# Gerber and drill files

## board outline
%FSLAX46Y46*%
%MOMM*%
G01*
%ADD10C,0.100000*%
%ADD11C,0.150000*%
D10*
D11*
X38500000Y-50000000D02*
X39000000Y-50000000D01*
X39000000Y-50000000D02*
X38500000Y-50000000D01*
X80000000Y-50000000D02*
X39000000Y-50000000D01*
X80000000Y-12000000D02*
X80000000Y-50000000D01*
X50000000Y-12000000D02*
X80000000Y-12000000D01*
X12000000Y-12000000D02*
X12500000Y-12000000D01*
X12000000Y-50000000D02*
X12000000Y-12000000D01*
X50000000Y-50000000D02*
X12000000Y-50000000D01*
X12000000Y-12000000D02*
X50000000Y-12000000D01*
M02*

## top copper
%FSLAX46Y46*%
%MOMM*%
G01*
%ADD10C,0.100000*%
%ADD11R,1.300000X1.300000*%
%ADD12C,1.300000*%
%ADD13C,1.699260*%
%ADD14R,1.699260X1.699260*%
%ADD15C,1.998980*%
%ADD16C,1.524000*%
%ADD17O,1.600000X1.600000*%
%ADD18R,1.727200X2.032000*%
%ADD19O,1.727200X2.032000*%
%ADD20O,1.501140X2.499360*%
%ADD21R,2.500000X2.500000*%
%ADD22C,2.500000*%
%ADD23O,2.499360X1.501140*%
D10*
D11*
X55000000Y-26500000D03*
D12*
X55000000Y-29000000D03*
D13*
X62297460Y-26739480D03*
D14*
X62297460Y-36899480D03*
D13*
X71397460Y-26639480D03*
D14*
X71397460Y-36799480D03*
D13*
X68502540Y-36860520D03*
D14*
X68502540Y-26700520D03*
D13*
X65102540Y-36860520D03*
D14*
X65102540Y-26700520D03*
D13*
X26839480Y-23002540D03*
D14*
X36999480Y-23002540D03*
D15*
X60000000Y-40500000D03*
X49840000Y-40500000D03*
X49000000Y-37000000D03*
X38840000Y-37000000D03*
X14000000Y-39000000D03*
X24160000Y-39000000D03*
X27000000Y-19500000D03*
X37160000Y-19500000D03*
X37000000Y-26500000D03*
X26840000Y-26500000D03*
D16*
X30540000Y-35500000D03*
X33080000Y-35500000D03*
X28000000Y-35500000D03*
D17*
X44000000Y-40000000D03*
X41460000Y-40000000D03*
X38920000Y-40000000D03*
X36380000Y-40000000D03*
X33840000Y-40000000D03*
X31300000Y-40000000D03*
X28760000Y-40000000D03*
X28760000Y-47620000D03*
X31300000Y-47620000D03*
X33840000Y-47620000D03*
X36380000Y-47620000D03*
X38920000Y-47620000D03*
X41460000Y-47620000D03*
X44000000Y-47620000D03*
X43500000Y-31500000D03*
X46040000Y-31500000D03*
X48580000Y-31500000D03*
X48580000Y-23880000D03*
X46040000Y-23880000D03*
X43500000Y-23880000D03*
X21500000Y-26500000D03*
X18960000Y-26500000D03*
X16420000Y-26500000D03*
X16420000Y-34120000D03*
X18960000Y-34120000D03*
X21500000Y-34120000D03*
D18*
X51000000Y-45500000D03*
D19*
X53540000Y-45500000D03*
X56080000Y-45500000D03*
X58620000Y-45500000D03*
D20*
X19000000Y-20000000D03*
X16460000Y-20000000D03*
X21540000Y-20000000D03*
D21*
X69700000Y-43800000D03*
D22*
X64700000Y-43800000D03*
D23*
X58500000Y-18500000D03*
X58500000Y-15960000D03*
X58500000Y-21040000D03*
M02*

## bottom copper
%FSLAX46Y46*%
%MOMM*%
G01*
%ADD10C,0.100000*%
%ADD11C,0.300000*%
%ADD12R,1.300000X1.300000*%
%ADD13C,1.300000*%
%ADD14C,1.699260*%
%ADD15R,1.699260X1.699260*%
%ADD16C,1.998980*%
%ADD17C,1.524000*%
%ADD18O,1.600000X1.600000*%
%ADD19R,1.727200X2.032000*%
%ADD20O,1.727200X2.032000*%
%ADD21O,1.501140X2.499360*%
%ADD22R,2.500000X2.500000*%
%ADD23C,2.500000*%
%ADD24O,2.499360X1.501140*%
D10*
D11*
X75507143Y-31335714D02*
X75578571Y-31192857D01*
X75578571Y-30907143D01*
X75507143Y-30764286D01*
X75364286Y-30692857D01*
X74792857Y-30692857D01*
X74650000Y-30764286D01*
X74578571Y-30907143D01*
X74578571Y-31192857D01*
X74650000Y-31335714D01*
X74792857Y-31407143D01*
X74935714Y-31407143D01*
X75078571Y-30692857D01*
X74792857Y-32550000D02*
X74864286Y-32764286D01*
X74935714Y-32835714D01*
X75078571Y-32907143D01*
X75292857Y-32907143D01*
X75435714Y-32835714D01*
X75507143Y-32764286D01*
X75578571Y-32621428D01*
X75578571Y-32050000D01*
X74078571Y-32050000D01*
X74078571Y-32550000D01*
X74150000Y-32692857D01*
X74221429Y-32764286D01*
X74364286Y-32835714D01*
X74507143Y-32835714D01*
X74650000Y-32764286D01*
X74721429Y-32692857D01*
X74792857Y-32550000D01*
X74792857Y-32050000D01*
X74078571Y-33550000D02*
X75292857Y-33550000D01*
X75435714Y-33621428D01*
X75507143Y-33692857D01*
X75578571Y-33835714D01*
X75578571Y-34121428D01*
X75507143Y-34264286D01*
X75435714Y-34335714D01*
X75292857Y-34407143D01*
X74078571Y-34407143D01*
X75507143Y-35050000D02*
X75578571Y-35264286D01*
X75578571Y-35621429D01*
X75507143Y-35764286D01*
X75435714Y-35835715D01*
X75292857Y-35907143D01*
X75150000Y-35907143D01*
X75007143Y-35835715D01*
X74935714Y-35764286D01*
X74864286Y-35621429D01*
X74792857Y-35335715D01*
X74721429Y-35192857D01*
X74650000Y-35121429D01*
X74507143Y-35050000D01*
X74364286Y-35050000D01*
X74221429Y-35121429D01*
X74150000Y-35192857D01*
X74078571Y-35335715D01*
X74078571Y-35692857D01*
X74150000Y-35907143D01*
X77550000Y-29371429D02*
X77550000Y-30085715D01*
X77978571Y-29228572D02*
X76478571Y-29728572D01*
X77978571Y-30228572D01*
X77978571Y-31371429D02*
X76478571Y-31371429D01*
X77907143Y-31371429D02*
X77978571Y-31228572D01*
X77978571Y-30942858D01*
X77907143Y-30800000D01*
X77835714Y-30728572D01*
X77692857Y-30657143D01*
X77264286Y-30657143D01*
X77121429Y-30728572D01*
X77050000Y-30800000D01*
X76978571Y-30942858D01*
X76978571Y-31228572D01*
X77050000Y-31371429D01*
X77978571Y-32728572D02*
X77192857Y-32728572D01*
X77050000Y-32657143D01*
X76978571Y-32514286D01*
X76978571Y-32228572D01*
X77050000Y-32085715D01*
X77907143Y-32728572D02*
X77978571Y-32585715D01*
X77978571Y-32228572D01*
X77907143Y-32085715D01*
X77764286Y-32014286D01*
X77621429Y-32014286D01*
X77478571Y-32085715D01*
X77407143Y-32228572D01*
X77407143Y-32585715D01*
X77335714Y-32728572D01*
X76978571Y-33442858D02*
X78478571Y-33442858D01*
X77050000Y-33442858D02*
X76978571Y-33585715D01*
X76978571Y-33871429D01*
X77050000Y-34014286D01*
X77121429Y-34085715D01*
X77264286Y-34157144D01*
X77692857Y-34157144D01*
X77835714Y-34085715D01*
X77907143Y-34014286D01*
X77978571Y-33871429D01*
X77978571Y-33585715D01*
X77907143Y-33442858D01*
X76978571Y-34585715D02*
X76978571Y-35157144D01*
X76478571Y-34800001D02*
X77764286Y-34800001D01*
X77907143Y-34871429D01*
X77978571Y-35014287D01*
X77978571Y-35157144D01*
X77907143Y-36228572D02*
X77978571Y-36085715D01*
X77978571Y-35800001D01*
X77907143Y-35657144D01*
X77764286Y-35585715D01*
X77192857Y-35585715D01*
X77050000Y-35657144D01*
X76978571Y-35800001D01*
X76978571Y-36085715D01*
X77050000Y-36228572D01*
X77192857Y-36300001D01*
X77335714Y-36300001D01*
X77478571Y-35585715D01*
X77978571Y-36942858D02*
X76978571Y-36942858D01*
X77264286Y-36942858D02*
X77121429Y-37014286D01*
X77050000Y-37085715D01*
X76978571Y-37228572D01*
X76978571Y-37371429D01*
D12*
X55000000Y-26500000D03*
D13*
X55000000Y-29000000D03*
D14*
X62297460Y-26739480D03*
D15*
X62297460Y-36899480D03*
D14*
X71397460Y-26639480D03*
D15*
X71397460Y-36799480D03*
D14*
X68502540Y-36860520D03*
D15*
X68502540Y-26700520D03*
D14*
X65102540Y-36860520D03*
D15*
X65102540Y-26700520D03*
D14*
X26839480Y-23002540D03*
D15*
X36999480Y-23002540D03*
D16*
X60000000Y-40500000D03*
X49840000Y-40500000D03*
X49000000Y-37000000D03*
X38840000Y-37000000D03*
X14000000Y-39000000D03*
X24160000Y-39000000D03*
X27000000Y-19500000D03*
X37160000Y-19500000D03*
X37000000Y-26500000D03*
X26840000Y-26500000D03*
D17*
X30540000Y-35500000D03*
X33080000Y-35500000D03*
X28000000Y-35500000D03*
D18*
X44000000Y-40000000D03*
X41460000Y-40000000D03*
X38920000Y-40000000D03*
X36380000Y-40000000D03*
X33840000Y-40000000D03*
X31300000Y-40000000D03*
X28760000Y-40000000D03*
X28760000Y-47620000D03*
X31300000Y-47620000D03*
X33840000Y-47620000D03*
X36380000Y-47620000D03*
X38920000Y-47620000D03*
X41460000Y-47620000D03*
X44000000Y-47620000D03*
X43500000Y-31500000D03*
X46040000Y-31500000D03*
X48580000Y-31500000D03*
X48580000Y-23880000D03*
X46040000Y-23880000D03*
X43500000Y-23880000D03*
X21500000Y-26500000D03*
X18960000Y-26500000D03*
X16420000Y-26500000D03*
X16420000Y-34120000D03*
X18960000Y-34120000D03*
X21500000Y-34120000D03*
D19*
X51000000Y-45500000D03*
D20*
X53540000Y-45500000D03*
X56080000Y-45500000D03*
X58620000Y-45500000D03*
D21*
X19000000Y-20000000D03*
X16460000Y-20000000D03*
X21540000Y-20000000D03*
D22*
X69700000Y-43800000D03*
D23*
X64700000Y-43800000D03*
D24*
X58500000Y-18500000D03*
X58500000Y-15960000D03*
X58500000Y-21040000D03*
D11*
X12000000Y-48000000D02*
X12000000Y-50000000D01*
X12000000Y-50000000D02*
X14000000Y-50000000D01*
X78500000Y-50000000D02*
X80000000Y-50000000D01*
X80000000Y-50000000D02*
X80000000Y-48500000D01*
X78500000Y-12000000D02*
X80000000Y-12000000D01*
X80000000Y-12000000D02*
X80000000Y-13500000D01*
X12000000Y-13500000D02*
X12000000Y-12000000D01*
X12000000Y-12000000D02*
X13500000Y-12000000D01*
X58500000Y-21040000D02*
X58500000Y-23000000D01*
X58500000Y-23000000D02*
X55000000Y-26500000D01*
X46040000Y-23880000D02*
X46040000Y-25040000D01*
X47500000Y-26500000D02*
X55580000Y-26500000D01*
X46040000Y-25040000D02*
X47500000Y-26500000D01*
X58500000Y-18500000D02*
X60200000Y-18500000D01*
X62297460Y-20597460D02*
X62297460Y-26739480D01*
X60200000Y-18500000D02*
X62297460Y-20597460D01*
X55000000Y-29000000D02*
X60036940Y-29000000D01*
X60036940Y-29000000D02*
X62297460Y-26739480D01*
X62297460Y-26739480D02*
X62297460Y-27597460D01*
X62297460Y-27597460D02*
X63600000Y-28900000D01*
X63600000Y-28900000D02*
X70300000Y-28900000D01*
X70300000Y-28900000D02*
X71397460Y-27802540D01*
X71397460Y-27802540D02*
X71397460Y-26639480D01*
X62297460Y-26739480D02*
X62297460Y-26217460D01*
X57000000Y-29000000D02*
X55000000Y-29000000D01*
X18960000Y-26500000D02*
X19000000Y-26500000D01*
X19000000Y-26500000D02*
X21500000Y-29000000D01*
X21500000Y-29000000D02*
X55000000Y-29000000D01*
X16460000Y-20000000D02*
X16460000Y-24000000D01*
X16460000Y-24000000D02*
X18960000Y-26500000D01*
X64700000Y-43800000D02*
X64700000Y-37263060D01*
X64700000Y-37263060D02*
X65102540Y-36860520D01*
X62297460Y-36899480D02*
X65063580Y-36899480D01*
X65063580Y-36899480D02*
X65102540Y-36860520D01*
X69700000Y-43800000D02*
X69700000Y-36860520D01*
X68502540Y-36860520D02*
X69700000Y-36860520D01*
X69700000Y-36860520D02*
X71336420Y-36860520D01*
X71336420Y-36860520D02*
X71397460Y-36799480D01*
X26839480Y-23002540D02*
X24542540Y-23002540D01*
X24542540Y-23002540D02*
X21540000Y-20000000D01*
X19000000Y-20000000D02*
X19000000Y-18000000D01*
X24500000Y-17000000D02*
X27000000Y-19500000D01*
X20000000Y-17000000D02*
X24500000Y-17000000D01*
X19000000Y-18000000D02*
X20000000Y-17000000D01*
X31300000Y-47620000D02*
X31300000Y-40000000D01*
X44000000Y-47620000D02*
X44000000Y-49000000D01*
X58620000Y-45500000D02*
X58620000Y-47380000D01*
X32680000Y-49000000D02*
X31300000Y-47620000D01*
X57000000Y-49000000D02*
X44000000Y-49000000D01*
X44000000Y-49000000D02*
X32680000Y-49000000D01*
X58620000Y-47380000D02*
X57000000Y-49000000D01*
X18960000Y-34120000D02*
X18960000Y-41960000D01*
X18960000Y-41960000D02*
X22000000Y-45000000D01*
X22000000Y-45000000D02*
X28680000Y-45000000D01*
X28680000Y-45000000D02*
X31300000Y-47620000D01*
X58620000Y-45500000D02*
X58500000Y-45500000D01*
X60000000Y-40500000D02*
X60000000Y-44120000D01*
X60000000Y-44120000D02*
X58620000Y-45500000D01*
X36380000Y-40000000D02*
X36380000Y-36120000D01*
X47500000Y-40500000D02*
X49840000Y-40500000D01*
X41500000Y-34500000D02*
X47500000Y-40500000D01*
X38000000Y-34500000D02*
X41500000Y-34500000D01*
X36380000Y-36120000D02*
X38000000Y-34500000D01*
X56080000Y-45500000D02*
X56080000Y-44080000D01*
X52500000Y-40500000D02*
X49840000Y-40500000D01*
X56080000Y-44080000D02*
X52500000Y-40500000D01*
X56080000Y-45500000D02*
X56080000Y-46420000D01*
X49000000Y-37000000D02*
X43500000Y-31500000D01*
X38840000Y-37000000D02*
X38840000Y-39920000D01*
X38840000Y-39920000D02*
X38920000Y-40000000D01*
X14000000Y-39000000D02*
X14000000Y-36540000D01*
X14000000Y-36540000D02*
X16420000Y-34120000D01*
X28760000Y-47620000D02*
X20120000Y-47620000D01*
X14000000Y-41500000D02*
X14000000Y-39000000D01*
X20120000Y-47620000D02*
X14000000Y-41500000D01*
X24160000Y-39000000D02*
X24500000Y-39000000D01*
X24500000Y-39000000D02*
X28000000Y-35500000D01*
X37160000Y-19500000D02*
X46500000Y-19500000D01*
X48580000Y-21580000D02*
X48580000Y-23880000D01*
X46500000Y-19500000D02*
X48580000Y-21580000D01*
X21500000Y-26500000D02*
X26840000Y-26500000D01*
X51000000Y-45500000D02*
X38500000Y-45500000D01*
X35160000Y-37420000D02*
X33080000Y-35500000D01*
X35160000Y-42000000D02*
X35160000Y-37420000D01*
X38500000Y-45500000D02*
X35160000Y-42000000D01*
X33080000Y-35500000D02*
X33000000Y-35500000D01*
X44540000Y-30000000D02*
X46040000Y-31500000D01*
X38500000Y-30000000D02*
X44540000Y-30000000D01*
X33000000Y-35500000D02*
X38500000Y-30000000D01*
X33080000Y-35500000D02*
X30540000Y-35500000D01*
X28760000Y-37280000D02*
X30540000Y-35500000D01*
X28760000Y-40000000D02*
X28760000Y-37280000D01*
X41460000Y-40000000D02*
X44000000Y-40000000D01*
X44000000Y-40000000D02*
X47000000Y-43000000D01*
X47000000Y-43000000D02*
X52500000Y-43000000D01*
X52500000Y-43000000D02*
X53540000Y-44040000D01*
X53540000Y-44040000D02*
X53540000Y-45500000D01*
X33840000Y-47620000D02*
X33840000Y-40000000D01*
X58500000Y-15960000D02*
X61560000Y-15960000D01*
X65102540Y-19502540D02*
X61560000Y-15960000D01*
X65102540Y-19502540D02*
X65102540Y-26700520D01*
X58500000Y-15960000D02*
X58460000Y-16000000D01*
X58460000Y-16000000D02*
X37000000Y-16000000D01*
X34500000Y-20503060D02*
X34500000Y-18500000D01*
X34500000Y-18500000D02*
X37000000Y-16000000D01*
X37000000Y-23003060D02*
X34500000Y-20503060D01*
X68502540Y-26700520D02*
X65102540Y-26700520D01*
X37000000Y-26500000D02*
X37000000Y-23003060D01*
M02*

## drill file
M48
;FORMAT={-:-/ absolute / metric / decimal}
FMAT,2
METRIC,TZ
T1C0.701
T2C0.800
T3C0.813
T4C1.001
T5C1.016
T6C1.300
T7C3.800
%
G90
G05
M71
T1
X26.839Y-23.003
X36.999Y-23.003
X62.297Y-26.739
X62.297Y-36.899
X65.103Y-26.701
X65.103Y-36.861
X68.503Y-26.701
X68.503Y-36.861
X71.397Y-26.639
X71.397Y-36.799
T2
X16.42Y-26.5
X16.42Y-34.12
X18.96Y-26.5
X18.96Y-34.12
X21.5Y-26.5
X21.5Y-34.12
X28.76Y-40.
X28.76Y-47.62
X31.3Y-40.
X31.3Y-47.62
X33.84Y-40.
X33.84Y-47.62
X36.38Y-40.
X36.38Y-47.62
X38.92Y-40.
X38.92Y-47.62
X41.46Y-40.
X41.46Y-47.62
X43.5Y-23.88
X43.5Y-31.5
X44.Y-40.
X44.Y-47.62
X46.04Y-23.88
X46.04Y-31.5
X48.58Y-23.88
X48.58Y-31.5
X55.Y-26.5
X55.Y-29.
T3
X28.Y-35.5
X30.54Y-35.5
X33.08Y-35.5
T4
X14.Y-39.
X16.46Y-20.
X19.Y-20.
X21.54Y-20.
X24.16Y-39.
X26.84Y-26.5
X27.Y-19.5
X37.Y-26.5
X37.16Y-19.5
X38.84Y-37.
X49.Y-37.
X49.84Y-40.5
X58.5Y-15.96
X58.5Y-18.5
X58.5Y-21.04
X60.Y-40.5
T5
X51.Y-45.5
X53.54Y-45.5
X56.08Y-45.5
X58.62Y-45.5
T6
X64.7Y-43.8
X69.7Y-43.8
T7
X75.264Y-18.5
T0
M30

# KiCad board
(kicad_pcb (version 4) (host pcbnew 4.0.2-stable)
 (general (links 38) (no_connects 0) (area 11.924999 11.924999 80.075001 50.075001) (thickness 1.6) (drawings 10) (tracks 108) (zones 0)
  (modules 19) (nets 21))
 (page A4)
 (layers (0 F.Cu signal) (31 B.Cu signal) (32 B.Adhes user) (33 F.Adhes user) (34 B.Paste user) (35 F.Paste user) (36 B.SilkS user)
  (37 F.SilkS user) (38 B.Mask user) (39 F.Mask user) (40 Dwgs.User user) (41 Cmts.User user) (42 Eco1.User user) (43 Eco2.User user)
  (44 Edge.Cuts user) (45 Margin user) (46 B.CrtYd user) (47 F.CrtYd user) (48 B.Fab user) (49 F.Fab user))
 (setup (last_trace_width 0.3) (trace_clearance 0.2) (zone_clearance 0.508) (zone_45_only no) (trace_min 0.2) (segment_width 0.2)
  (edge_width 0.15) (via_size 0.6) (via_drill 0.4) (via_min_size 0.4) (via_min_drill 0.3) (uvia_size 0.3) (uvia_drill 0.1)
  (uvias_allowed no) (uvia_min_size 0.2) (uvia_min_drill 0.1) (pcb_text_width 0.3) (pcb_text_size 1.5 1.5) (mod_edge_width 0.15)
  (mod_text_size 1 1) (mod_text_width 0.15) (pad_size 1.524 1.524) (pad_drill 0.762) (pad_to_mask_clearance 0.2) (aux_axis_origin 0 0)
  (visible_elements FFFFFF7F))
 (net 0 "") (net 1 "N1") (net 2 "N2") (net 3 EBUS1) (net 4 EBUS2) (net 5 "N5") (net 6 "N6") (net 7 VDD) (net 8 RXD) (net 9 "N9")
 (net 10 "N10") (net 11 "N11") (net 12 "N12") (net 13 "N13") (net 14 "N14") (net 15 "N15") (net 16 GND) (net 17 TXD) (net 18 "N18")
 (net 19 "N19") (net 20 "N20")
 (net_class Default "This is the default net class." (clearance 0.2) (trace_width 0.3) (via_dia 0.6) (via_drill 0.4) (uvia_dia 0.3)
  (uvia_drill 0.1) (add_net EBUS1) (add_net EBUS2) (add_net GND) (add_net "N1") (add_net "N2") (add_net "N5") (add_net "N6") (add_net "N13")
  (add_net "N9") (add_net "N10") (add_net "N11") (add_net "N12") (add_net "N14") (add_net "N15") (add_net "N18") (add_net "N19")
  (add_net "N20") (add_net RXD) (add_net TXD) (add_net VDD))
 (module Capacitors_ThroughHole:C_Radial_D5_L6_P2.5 (layer F.Cu) (at 55 26.5 270)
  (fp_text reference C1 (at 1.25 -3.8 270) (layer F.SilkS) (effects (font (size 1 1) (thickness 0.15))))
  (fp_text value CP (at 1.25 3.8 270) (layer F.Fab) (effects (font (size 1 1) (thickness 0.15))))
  (pad 1 thru_hole rect (at 0 0 270) (size 1.3 1.3) (drill 0.8) (layers *.Cu *.Mask F.SilkS) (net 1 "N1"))
  (pad 2 thru_hole circle (at 2.5 0 270) (size 1.3 1.3) (drill 0.8) (layers *.Cu *.Mask F.SilkS) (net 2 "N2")))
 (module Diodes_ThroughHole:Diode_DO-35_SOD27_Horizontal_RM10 (layer F.Cu) (at 62.3 36.9 90)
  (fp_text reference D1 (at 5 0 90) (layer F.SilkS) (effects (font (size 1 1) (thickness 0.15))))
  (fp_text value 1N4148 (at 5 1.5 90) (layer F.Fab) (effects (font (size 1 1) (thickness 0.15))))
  (pad 2 thru_hole circle (at 10.16052 -0.00254 270) (size 1.69926 1.69926) (drill 0.70104) (layers *.Cu *.Mask F.SilkS) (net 2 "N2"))
  (pad 1 thru_hole rect (at 0.00052 -0.00254 270) (size 1.69926 1.69926) (drill 0.70104) (layers *.Cu *.Mask F.SilkS) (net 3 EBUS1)))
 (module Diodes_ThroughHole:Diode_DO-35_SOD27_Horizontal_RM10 (layer F.Cu) (at 71.4 36.8 90)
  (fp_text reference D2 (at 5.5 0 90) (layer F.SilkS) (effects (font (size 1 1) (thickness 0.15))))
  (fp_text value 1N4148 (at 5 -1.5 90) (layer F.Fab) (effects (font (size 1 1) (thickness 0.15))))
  (pad 2 thru_hole circle (at 10.16052 -0.00254 270) (size 1.69926 1.69926) (drill 0.70104) (layers *.Cu *.Mask F.SilkS) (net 2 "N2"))
  (pad 1 thru_hole rect (at 0.00052 -0.00254 270) (size 1.69926 1.69926) (drill 0.70104) (layers *.Cu *.Mask F.SilkS) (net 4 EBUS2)))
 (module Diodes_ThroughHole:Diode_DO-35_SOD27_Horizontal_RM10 (layer F.Cu) (at 68.5 26.7 270)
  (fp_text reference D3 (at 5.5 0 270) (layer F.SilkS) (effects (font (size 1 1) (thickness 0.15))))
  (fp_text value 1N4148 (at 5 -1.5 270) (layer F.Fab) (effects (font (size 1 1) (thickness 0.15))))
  (pad 2 thru_hole circle (at 10.16052 -0.00254 90) (size 1.69926 1.69926) (drill 0.70104) (layers *.Cu *.Mask F.SilkS) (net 4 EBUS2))
  (pad 1 thru_hole rect (at 0.00052 -0.00254 90) (size 1.69926 1.69926) (drill 0.70104) (layers *.Cu *.Mask F.SilkS) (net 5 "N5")))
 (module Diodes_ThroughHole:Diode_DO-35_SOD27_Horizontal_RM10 (layer F.Cu) (at 65.1 26.7 270)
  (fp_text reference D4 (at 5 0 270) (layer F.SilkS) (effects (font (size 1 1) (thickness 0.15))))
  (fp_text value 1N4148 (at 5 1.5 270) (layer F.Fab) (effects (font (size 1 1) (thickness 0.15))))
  (pad 2 thru_hole circle (at 10.16052 -0.00254 90) (size 1.69926 1.69926) (drill 0.70104) (layers *.Cu *.Mask F.SilkS) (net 3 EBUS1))
  (pad 1 thru_hole rect (at 0.00052 -0.00254 90) (size 1.69926 1.69926) (drill 0.70104) (layers *.Cu *.Mask F.SilkS) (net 5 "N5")))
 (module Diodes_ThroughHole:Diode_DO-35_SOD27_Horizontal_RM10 (layer F.Cu) (at 37 23 180)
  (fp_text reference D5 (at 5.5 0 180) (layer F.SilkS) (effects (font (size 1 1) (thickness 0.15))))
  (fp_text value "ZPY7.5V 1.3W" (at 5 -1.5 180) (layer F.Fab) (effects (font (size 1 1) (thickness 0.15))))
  (pad 2 thru_hole circle (at 10.16052 -0.00254) (size 1.69926 1.69926) (drill 0.70104) (layers *.Cu *.Mask F.SilkS) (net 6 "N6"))
  (pad 1 thru_hole rect (at 0.00052 -0.00254) (size 1.69926 1.69926) (drill 0.70104) (layers *.Cu *.Mask F.SilkS) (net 5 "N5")))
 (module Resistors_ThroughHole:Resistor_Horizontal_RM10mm (layer F.Cu) (at 60 40.5 180)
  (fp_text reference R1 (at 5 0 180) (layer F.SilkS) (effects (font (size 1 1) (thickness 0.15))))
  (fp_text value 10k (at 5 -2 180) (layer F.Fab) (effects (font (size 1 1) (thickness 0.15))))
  (pad 1 thru_hole circle (at 0 0 180) (size 1.99898 1.99898) (drill 1.00076) (layers *.Cu *.SilkS *.Mask) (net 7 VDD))
  (pad 2 thru_hole circle (at 10.16 0 180) (size 1.99898 1.99898) (drill 1.00076) (layers *.Cu *.SilkS *.Mask) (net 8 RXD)))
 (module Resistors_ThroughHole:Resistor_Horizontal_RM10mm (layer F.Cu) (at 49 37 180)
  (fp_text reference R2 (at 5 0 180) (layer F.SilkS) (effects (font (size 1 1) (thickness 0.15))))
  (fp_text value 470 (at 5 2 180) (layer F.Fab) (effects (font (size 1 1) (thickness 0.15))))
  (pad 1 thru_hole circle (at 0 0 180) (size 1.99898 1.99898) (drill 1.00076) (layers *.Cu *.SilkS *.Mask) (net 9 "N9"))
  (pad 2 thru_hole circle (at 10.16 0 180) (size 1.99898 1.99898) (drill 1.00076) (layers *.Cu *.SilkS *.Mask) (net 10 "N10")))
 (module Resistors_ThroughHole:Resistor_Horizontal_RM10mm (layer F.Cu) (at 14 39)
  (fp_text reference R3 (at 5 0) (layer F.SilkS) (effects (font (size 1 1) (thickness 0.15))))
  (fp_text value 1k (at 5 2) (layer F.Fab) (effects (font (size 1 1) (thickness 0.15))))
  (pad 1 thru_hole circle (at 0 0) (size 1.99898 1.99898) (drill 1.00076) (layers *.Cu *.SilkS *.Mask) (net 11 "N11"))
  (pad 2 thru_hole circle (at 10.16 0) (size 1.99898 1.99898) (drill 1.00076) (layers *.Cu *.SilkS *.Mask) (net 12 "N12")))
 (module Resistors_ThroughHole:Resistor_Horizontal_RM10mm (layer F.Cu) (at 27 19.5)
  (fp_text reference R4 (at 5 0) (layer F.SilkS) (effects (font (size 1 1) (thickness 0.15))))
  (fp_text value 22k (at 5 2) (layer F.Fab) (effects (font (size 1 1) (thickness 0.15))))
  (pad 1 thru_hole circle (at 0 0) (size 1.99898 1.99898) (drill 1.00076) (layers *.Cu *.SilkS *.Mask) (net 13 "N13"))
  (pad 2 thru_hole circle (at 10.16 0) (size 1.99898 1.99898) (drill 1.00076) (layers *.Cu *.SilkS *.Mask) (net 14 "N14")))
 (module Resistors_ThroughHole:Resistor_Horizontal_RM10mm (layer F.Cu) (at 37 26.5 180)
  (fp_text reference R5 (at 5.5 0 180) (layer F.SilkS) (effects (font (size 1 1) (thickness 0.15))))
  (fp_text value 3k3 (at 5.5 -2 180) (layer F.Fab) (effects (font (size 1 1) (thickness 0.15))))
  (pad 1 thru_hole circle (at 0 0 180) (size 1.99898 1.99898) (drill 1.00076) (layers *.Cu *.SilkS *.Mask) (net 5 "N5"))
  (pad 2 thru_hole circle (at 10.16 0 180) (size 1.99898 1.99898) (drill 1.00076) (layers *.Cu *.SilkS *.Mask) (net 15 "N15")))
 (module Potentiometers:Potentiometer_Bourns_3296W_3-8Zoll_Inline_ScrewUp (layer F.Cu) (at 28 35.5 270)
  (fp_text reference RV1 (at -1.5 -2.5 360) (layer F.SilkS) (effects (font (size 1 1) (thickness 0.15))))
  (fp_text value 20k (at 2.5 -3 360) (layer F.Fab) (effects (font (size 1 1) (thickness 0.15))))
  (pad 2 thru_hole circle (at 0 -2.54 270) (size 1.524 1.524) (drill 0.8128) (layers *.Cu *.Mask F.SilkS) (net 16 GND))
  (pad 3 thru_hole circle (at 0 -5.08 270) (size 1.524 1.524) (drill 0.8128) (layers *.Cu *.Mask F.SilkS) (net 16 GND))
  (pad 1 thru_hole circle (at 0 0 270) (size 1.524 1.524) (drill 0.8128) (layers *.Cu *.Mask F.SilkS) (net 12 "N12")))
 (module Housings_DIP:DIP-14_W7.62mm (layer F.Cu) (at 44 40 270)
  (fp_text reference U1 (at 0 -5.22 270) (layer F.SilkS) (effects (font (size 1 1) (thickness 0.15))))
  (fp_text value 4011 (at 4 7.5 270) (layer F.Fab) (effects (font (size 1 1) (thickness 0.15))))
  (pad 1 thru_hole oval (at 0 0 270) (size 1.6 1.6) (drill 0.8) (layers *.Cu *.Mask F.SilkS) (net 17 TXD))
  (pad 2 thru_hole oval (at 0 2.54 270) (size 1.6 1.6) (drill 0.8) (layers *.Cu *.Mask F.SilkS) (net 17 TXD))
  (pad 3 thru_hole oval (at 0 5.08 270) (size 1.6 1.6) (drill 0.8) (layers *.Cu *.Mask F.SilkS) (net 10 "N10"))
  (pad 4 thru_hole oval (at 0 7.62 270) (size 1.6 1.6) (drill 0.8) (layers *.Cu *.Mask F.SilkS) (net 8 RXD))
  (pad 5 thru_hole oval (at 0 10.16 270) (size 1.6 1.6) (drill 0.8) (layers *.Cu *.Mask F.SilkS) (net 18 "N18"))
  (pad 6 thru_hole oval (at 0 12.7 270) (size 1.6 1.6) (drill 0.8) (layers *.Cu *.Mask F.SilkS) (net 7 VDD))
  (pad 7 thru_hole oval (at 0 15.24 270) (size 1.6 1.6) (drill 0.8) (layers *.Cu *.Mask F.SilkS) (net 16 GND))
  (pad 8 thru_hole oval (at 7.62 15.24 270) (size 1.6 1.6) (drill 0.8) (layers *.Cu *.Mask F.SilkS) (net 11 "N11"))
  (pad 9 thru_hole oval (at 7.62 12.7 270) (size 1.6 1.6) (drill 0.8) (layers *.Cu *.Mask F.SilkS) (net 7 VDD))
  (pad 10 thru_hole oval (at 7.62 10.16 270) (size 1.6 1.6) (drill 0.8) (layers *.Cu *.Mask F.SilkS) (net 18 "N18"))
  (pad 11 thru_hole oval (at 7.62 7.62 270) (size 1.6 1.6) (drill 0.8) (layers *.Cu *.Mask F.SilkS))
  (pad 12 thru_hole oval (at 7.62 5.08 270) (size 1.6 1.6) (drill 0.8) (layers *.Cu *.Mask F.SilkS))
  (pad 13 thru_hole oval (at 7.62 2.54 270) (size 1.6 1.6) (drill 0.8) (layers *.Cu *.Mask F.SilkS))
  (pad 14 thru_hole oval (at 7.62 0 270) (size 1.6 1.6) (drill 0.8) (layers *.Cu *.Mask F.SilkS) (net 7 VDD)))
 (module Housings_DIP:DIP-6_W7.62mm (layer F.Cu) (at 43.5 31.5 90)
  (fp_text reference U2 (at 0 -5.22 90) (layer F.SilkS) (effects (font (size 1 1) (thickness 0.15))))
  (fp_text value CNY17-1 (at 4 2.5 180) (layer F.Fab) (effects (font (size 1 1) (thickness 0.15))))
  (pad 1 thru_hole oval (at 0 0 90) (size 1.6 1.6) (drill 0.8) (layers *.Cu *.Mask F.SilkS) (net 9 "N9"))
  (pad 2 thru_hole oval (at 0 2.54 90) (size 1.6 1.6) (drill 0.8) (layers *.Cu *.Mask F.SilkS) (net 16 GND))
  (pad 3 thru_hole oval (at 0 5.08 90) (size 1.6 1.6) (drill 0.8) (layers *.Cu *.Mask F.SilkS))
  (pad 4 thru_hole oval (at 7.62 5.08 90) (size 1.6 1.6) (drill 0.8) (layers *.Cu *.Mask F.SilkS) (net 14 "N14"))
  (pad 5 thru_hole oval (at 7.62 2.54 90) (size 1.6 1.6) (drill 0.8) (layers *.Cu *.Mask F.SilkS) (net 1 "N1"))
  (pad 6 thru_hole oval (at 7.62 0 90) (size 1.6 1.6) (drill 0.8) (layers *.Cu *.Mask F.SilkS) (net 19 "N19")))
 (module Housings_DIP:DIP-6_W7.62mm (layer F.Cu) (at 21.5 26.5 270)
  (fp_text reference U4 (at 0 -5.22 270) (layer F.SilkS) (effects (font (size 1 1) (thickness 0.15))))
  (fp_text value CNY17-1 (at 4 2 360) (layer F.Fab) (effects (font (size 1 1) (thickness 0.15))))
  (pad 1 thru_hole oval (at 0 0 270) (size 1.6 1.6) (drill 0.8) (layers *.Cu *.Mask F.SilkS) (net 15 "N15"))
  (pad 2 thru_hole oval (at 0 2.54 270) (size 1.6 1.6) (drill 0.8) (layers *.Cu *.Mask F.SilkS) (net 2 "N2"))
  (pad 3 thru_hole oval (at 0 5.08 270) (size 1.6 1.6) (drill 0.8) (layers *.Cu *.Mask F.SilkS))
  (pad 4 thru_hole oval (at 7.62 5.08 270) (size 1.6 1.6) (drill 0.8) (layers *.Cu *.Mask F.SilkS) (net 11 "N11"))
  (pad 5 thru_hole oval (at 7.62 2.54 270) (size 1.6 1.6) (drill 0.8) (layers *.Cu *.Mask F.SilkS) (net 7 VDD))
  (pad 6 thru_hole oval (at 7.62 0 270) (size 1.6 1.6) (drill 0.8) (layers *.Cu *.Mask F.SilkS) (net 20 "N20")))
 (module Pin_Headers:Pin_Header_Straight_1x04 (layer F.Cu) (at 51 45.5 90)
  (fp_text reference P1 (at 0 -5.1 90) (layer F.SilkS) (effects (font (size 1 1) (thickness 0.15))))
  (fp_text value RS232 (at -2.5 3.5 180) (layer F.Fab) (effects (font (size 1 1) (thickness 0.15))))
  (pad 1 thru_hole rect (at 0 0 90) (size 2.032 1.7272) (drill 1.016) (layers *.Cu *.Mask F.SilkS) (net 16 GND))
  (pad 2 thru_hole oval (at 0 2.54 90) (size 2.032 1.7272) (drill 1.016) (layers *.Cu *.Mask F.SilkS) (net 17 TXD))
  (pad 3 thru_hole oval (at 0 5.08 90) (size 2.032 1.7272) (drill 1.016) (layers *.Cu *.Mask F.SilkS) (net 8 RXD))
  (pad 4 thru_hole oval (at 0 7.62 90) (size 2.032 1.7272) (drill 1.016) (layers *.Cu *.Mask F.SilkS) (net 7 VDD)))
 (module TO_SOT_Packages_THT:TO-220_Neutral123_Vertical (layer F.Cu) (at 19 20)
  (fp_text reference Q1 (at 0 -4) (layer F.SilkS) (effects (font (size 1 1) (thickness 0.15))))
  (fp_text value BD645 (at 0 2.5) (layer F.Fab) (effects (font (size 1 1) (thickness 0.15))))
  (pad 2 thru_hole oval (at 0 0 90) (size 2.49936 1.50114) (drill 1.00076) (layers *.Cu *.Mask F.SilkS) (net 13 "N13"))
  (pad 1 thru_hole oval (at -2.54 0 90) (size 2.49936 1.50114) (drill 1.00076) (layers *.Cu *.Mask F.SilkS) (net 2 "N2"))
  (pad 3 thru_hole oval (at 2.54 0 90) (size 2.49936 1.50114) (drill 1.00076) (layers *.Cu *.Mask F.SilkS) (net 6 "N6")))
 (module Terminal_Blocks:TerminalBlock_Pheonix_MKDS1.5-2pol (layer F.Cu) (at 69.7 43.8 180)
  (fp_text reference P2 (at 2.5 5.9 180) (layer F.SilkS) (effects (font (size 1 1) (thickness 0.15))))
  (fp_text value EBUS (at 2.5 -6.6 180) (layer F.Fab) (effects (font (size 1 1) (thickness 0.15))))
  (pad 1 thru_hole rect (at 0 0 180) (size 2.5 2.5) (drill 1.3) (layers *.Cu *.Mask F.SilkS) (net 4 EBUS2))
  (pad 2 thru_hole circle (at 5 0 180) (size 2.5 2.5) (drill 1.3) (layers *.Cu *.Mask F.SilkS) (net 3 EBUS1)))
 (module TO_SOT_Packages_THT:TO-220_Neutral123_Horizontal (layer F.Cu) (at 58.5 18.5 270)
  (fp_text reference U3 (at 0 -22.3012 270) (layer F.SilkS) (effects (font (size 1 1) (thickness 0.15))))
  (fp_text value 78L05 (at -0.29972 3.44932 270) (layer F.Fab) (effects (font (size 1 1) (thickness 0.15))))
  (pad 2 thru_hole oval (at 0 0) (size 2.49936 1.50114) (drill 1.00076) (layers *.Cu *.Mask F.SilkS) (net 2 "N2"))
  (pad 1 thru_hole oval (at -2.54 0) (size 2.49936 1.50114) (drill 1.00076) (layers *.Cu *.Mask F.SilkS) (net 5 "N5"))
  (pad 3 thru_hole oval (at 2.54 0) (size 2.49936 1.50114) (drill 1.00076) (layers *.Cu *.Mask F.SilkS) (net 1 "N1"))
  (pad "" np_thru_hole circle (at 0 -16.764) (size 3.79984 3.79984) (drill 3.79984) (layers *.Cu *.Mask F.SilkS)))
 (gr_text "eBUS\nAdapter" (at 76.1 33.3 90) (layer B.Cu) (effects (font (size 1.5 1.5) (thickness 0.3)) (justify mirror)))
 (gr_line (start 38.5 50) (end 39 50) (angle 90) (layer Edge.Cuts) (width 0.15))
 (gr_line (start 39 50) (end 38.5 50) (angle 90) (layer Edge.Cuts) (width 0.15))
 (gr_line (start 80 50) (end 39 50) (angle 90) (layer Edge.Cuts) (width 0.15))
 (gr_line (start 80 12) (end 80 50) (angle 90) (layer Edge.Cuts) (width 0.15))
 (gr_line (start 50 12) (end 80 12) (angle 90) (layer Edge.Cuts) (width 0.15))
 (gr_line (start 12 12) (end 12.5 12) (angle 90) (layer Edge.Cuts) (width 0.15))
 (gr_line (start 12 50) (end 12 12) (angle 90) (layer Edge.Cuts) (width 0.15))
 (gr_line (start 50 50) (end 12 50) (angle 90) (layer Edge.Cuts) (width 0.15))
 (gr_line (start 12 12) (end 50 12) (angle 90) (layer Edge.Cuts) (width 0.15))
 (segment (start 12 48) (end 12 50) (width 0.3) (layer B.Cu) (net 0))
 (segment (start 12 50) (end 14 50) (width 0.3) (layer B.Cu) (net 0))
 (segment (start 78.5 50) (end 80 50) (width 0.3) (layer B.Cu) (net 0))
 (segment (start 80 50) (end 80 48.5) (width 0.3) (layer B.Cu) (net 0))
 (segment (start 78.5 12) (end 80 12) (width 0.3) (layer B.Cu) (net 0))
 (segment (start 80 12) (end 80 13.5) (width 0.3) (layer B.Cu) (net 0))
 (segment (start 12 13.5) (end 12 12) (width 0.3) (layer B.Cu) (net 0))
 (segment (start 12 12) (end 13.5 12) (width 0.3) (layer B.Cu) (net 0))
 (segment (start 58.5 21.04) (end 58.5 23) (width 0.3) (layer B.Cu) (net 1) (status 400000))
 (segment (start 58.5 23) (end 55 26.5) (width 0.3) (layer B.Cu) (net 1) (status 800000))
 (segment (start 46.04 23.88) (end 46.04 25.04) (width 0.3) (layer B.Cu) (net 1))
 (segment (start 47.5 26.5) (end 55.58 26.5) (width 0.3) (layer B.Cu) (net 1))
 (segment (start 46.04 25.04) (end 47.5 26.5) (width 0.3) (layer B.Cu) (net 1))
 (segment (start 58.5 18.5) (end 60.2 18.5) (width 0.3) (layer B.Cu) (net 2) (status 400000))
 (segment (start 62.29746 20.59746) (end 62.29746 26.73948) (width 0.3) (layer B.Cu) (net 2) (status 800000))
 (segment (start 60.2 18.5) (end 62.29746 20.59746) (width 0.3) (layer B.Cu) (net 2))
 (segment (start 55 29) (end 60.03694 29) (width 0.3) (layer B.Cu) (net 2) (status 400000))
 (segment (start 60.03694 29) (end 62.29746 26.73948) (width 0.3) (layer B.Cu) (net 2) (status 800000))
 (segment (start 62.29746 26.73948) (end 62.29746 27.59746) (width 0.3) (layer B.Cu) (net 2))
 (segment (start 62.29746 27.59746) (end 63.6 28.9) (width 0.3) (layer B.Cu) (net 2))
 (segment (start 63.6 28.9) (end 70.3 28.9) (width 0.3) (layer B.Cu) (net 2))
 (segment (start 70.3 28.9) (end 71.39746 27.80254) (width 0.3) (layer B.Cu) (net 2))
 (segment (start 71.39746 27.80254) (end 71.39746 26.63948) (width 0.3) (layer B.Cu) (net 2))
 (segment (start 62.29746 26.73948) (end 62.29746 26.21746) (width 0.3) (layer B.Cu) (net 2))
 (segment (start 57 29) (end 55 29) (width 0.3) (layer B.Cu) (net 2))
 (segment (start 18.96 26.5) (end 19 26.5) (width 0.3) (layer B.Cu) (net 2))
 (segment (start 19 26.5) (end 21.5 29) (width 0.3) (layer B.Cu) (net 2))
 (segment (start 21.5 29) (end 55 29) (width 0.3) (layer B.Cu) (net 2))
 (segment (start 16.46 20) (end 16.46 24) (width 0.3) (layer B.Cu) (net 2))
 (segment (start 16.46 24) (end 18.96 26.5) (width 0.3) (layer B.Cu) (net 2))
 (segment (start 64.7 43.8) (end 64.7 37.26306) (width 0.3) (layer B.Cu) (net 3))
 (segment (start 64.7 37.26306) (end 65.10254 36.86052) (width 0.3) (layer B.Cu) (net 3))
 (segment (start 62.29746 36.89948) (end 65.06358 36.89948) (width 0.3) (layer B.Cu) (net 3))
 (segment (start 65.06358 36.89948) (end 65.10254 36.86052) (width 0.3) (layer B.Cu) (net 3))
 (segment (start 69.7 43.8) (end 69.7 36.86052) (width 0.3) (layer B.Cu) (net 4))
 (segment (start 68.50254 36.86052) (end 69.7 36.86052) (width 0.3) (layer B.Cu) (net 4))
 (segment (start 69.7 36.86052) (end 71.33642 36.86052) (width 0.3) (layer B.Cu) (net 4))
 (segment (start 71.33642 36.86052) (end 71.39746 36.79948) (width 0.3) (layer B.Cu) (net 4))
 (segment (start 26.83948 23.00254) (end 24.54254 23.00254) (width 0.3) (layer B.Cu) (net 6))
 (segment (start 24.54254 23.00254) (end 21.54 20) (width 0.3) (layer B.Cu) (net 6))
 (segment (start 19 20) (end 19 18) (width 0.3) (layer B.Cu) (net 13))
 (segment (start 24.5 17) (end 27 19.5) (width 0.3) (layer B.Cu) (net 13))
 (segment (start 20 17) (end 24.5 17) (width 0.3) (layer B.Cu) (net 13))
 (segment (start 19 18) (end 20 17) (width 0.3) (layer B.Cu) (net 13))
 (segment (start 31.3 47.62) (end 31.3 40) (width 0.3) (layer B.Cu) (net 7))
 (segment (start 44 47.62) (end 44 49) (width 0.3) (layer B.Cu) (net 7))
 (segment (start 58.62 45.5) (end 58.62 47.38) (width 0.3) (layer B.Cu) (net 7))
 (segment (start 32.68 49) (end 31.3 47.62) (width 0.3) (layer B.Cu) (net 7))
 (segment (start 57 49) (end 44 49) (width 0.3) (layer B.Cu) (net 7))
 (segment (start 44 49) (end 32.68 49) (width 0.3) (layer B.Cu) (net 7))
 (segment (start 58.62 47.38) (end 57 49) (width 0.3) (layer B.Cu) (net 7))
 (segment (start 18.96 34.12) (end 18.96 41.96) (width 0.3) (layer B.Cu) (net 7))
 (segment (start 18.96 41.96) (end 22 45) (width 0.3) (layer B.Cu) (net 7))
 (segment (start 22 45) (end 28.68 45) (width 0.3) (layer B.Cu) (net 7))
 (segment (start 28.68 45) (end 31.3 47.62) (width 0.3) (layer B.Cu) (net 7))
 (segment (start 58.62 45.5) (end 58.5 45.5) (width 0.3) (layer B.Cu) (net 7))
 (segment (start 60 40.5) (end 60 44.12) (width 0.3) (layer B.Cu) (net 7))
 (segment (start 60 44.12) (end 58.62 45.5) (width 0.3) (layer B.Cu) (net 7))
 (segment (start 36.38 40) (end 36.38 36.12) (width 0.3) (layer B.Cu) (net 8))
 (segment (start 47.5 40.5) (end 49.84 40.5) (width 0.3) (layer B.Cu) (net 8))
 (segment (start 41.5 34.5) (end 47.5 40.5) (width 0.3) (layer B.Cu) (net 8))
 (segment (start 38 34.5) (end 41.5 34.5) (width 0.3) (layer B.Cu) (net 8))
 (segment (start 36.38 36.12) (end 38 34.5) (width 0.3) (layer B.Cu) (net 8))
 (segment (start 56.08 45.5) (end 56.08 44.08) (width 0.3) (layer B.Cu) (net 8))
 (segment (start 52.5 40.5) (end 49.84 40.5) (width 0.3) (layer B.Cu) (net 8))
 (segment (start 56.08 44.08) (end 52.5 40.5) (width 0.3) (layer B.Cu) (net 8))
 (segment (start 56.08 45.5) (end 56.08 46.42) (width 0.3) (layer B.Cu) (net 8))
 (segment (start 49 37) (end 43.5 31.5) (width 0.3) (layer B.Cu) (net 9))
 (segment (start 38.84 37) (end 38.84 39.92) (width 0.3) (layer B.Cu) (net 10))
 (segment (start 38.84 39.92) (end 38.92 40) (width 0.3) (layer B.Cu) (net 10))
 (segment (start 14 39) (end 14 36.54) (width 0.3) (layer B.Cu) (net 11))
 (segment (start 14 36.54) (end 16.42 34.12) (width 0.3) (layer B.Cu) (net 11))
 (segment (start 28.76 47.62) (end 20.12 47.62) (width 0.3) (layer B.Cu) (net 11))
 (segment (start 14 41.5) (end 14 39) (width 0.3) (layer B.Cu) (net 11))
 (segment (start 20.12 47.62) (end 14 41.5) (width 0.3) (layer B.Cu) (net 11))
 (segment (start 24.16 39) (end 24.5 39) (width 0.3) (layer B.Cu) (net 12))
 (segment (start 24.5 39) (end 28 35.5) (width 0.3) (layer B.Cu) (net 12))
 (segment (start 37.16 19.5) (end 46.5 19.5) (width 0.3) (layer B.Cu) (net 14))
 (segment (start 48.58 21.58) (end 48.58 23.88) (width 0.3) (layer B.Cu) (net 14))
 (segment (start 46.5 19.5) (end 48.58 21.58) (width 0.3) (layer B.Cu) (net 14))
 (segment (start 21.5 26.5) (end 26.84 26.5) (width 0.3) (layer B.Cu) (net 15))
 (segment (start 51 45.5) (end 38.5 45.5) (width 0.3) (layer B.Cu) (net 16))
 (segment (start 35.16 37.42) (end 33.08 35.5) (width 0.3) (layer B.Cu) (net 16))
 (segment (start 35.16 42) (end 35.16 37.42) (width 0.3) (layer B.Cu) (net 16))
 (segment (start 38.5 45.5) (end 35.16 42) (width 0.3) (layer B.Cu) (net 16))
 (segment (start 33.08 35.5) (end 33 35.5) (width 0.3) (layer B.Cu) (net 16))
 (segment (start 44.54 30) (end 46.04 31.5) (width 0.3) (layer B.Cu) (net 16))
 (segment (start 38.5 30) (end 44.54 30) (width 0.3) (layer B.Cu) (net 16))
 (segment (start 33 35.5) (end 38.5 30) (width 0.3) (layer B.Cu) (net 16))
 (segment (start 33.08 35.5) (end 30.54 35.5) (width 0.3) (layer B.Cu) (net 16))
 (segment (start 28.76 37.28) (end 30.54 35.5) (width 0.3) (layer B.Cu) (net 16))
 (segment (start 28.76 40) (end 28.76 37.28) (width 0.3) (layer B.Cu) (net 16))
 (segment (start 41.46 40) (end 44 40) (width 0.3) (layer B.Cu) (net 17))
 (segment (start 44 40) (end 47 43) (width 0.3) (layer B.Cu) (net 17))
 (segment (start 47 43) (end 52.5 43) (width 0.3) (layer B.Cu) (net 17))
 (segment (start 52.5 43) (end 53.54 44.04) (width 0.3) (layer B.Cu) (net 17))
 (segment (start 53.54 44.04) (end 53.54 45.5) (width 0.3) (layer B.Cu) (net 17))
 (segment (start 33.84 47.62) (end 33.84 40) (width 0.3) (layer B.Cu) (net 18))
 (segment (start 58.5 15.96) (end 61.56 15.96) (width 0.3) (layer B.Cu) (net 5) (status 400000))
 (segment (start 65.10254 19.50254) (end 61.56 15.96) (width 0.3) (layer B.Cu) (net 5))
 (segment (start 65.10254 19.50254) (end 65.10254 26.70052) (width 0.3) (layer B.Cu) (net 5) (status 800000))
 (segment (start 58.5 15.96) (end 58.46 16) (width 0.3) (layer B.Cu) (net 5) (status C00000))
 (segment (start 58.46 16) (end 37 16) (width 0.3) (layer B.Cu) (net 5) (status 400000))
 (segment (start 34.5 20.50306) (end 34.5 18.5) (width 0.3) (layer B.Cu) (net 5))
 (segment (start 34.5 18.5) (end 37 16) (width 0.3) (layer B.Cu) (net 5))
 (segment (start 37 23.00306) (end 34.5 20.50306) (width 0.3) (layer B.Cu) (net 5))
 (segment (start 68.50254 26.70052) (end 65.10254 26.70052) (width 0.3) (layer B.Cu) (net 5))
 (segment (start 37 26.5) (end 37 23.00306) (width 0.3) (layer B.Cu) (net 5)))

